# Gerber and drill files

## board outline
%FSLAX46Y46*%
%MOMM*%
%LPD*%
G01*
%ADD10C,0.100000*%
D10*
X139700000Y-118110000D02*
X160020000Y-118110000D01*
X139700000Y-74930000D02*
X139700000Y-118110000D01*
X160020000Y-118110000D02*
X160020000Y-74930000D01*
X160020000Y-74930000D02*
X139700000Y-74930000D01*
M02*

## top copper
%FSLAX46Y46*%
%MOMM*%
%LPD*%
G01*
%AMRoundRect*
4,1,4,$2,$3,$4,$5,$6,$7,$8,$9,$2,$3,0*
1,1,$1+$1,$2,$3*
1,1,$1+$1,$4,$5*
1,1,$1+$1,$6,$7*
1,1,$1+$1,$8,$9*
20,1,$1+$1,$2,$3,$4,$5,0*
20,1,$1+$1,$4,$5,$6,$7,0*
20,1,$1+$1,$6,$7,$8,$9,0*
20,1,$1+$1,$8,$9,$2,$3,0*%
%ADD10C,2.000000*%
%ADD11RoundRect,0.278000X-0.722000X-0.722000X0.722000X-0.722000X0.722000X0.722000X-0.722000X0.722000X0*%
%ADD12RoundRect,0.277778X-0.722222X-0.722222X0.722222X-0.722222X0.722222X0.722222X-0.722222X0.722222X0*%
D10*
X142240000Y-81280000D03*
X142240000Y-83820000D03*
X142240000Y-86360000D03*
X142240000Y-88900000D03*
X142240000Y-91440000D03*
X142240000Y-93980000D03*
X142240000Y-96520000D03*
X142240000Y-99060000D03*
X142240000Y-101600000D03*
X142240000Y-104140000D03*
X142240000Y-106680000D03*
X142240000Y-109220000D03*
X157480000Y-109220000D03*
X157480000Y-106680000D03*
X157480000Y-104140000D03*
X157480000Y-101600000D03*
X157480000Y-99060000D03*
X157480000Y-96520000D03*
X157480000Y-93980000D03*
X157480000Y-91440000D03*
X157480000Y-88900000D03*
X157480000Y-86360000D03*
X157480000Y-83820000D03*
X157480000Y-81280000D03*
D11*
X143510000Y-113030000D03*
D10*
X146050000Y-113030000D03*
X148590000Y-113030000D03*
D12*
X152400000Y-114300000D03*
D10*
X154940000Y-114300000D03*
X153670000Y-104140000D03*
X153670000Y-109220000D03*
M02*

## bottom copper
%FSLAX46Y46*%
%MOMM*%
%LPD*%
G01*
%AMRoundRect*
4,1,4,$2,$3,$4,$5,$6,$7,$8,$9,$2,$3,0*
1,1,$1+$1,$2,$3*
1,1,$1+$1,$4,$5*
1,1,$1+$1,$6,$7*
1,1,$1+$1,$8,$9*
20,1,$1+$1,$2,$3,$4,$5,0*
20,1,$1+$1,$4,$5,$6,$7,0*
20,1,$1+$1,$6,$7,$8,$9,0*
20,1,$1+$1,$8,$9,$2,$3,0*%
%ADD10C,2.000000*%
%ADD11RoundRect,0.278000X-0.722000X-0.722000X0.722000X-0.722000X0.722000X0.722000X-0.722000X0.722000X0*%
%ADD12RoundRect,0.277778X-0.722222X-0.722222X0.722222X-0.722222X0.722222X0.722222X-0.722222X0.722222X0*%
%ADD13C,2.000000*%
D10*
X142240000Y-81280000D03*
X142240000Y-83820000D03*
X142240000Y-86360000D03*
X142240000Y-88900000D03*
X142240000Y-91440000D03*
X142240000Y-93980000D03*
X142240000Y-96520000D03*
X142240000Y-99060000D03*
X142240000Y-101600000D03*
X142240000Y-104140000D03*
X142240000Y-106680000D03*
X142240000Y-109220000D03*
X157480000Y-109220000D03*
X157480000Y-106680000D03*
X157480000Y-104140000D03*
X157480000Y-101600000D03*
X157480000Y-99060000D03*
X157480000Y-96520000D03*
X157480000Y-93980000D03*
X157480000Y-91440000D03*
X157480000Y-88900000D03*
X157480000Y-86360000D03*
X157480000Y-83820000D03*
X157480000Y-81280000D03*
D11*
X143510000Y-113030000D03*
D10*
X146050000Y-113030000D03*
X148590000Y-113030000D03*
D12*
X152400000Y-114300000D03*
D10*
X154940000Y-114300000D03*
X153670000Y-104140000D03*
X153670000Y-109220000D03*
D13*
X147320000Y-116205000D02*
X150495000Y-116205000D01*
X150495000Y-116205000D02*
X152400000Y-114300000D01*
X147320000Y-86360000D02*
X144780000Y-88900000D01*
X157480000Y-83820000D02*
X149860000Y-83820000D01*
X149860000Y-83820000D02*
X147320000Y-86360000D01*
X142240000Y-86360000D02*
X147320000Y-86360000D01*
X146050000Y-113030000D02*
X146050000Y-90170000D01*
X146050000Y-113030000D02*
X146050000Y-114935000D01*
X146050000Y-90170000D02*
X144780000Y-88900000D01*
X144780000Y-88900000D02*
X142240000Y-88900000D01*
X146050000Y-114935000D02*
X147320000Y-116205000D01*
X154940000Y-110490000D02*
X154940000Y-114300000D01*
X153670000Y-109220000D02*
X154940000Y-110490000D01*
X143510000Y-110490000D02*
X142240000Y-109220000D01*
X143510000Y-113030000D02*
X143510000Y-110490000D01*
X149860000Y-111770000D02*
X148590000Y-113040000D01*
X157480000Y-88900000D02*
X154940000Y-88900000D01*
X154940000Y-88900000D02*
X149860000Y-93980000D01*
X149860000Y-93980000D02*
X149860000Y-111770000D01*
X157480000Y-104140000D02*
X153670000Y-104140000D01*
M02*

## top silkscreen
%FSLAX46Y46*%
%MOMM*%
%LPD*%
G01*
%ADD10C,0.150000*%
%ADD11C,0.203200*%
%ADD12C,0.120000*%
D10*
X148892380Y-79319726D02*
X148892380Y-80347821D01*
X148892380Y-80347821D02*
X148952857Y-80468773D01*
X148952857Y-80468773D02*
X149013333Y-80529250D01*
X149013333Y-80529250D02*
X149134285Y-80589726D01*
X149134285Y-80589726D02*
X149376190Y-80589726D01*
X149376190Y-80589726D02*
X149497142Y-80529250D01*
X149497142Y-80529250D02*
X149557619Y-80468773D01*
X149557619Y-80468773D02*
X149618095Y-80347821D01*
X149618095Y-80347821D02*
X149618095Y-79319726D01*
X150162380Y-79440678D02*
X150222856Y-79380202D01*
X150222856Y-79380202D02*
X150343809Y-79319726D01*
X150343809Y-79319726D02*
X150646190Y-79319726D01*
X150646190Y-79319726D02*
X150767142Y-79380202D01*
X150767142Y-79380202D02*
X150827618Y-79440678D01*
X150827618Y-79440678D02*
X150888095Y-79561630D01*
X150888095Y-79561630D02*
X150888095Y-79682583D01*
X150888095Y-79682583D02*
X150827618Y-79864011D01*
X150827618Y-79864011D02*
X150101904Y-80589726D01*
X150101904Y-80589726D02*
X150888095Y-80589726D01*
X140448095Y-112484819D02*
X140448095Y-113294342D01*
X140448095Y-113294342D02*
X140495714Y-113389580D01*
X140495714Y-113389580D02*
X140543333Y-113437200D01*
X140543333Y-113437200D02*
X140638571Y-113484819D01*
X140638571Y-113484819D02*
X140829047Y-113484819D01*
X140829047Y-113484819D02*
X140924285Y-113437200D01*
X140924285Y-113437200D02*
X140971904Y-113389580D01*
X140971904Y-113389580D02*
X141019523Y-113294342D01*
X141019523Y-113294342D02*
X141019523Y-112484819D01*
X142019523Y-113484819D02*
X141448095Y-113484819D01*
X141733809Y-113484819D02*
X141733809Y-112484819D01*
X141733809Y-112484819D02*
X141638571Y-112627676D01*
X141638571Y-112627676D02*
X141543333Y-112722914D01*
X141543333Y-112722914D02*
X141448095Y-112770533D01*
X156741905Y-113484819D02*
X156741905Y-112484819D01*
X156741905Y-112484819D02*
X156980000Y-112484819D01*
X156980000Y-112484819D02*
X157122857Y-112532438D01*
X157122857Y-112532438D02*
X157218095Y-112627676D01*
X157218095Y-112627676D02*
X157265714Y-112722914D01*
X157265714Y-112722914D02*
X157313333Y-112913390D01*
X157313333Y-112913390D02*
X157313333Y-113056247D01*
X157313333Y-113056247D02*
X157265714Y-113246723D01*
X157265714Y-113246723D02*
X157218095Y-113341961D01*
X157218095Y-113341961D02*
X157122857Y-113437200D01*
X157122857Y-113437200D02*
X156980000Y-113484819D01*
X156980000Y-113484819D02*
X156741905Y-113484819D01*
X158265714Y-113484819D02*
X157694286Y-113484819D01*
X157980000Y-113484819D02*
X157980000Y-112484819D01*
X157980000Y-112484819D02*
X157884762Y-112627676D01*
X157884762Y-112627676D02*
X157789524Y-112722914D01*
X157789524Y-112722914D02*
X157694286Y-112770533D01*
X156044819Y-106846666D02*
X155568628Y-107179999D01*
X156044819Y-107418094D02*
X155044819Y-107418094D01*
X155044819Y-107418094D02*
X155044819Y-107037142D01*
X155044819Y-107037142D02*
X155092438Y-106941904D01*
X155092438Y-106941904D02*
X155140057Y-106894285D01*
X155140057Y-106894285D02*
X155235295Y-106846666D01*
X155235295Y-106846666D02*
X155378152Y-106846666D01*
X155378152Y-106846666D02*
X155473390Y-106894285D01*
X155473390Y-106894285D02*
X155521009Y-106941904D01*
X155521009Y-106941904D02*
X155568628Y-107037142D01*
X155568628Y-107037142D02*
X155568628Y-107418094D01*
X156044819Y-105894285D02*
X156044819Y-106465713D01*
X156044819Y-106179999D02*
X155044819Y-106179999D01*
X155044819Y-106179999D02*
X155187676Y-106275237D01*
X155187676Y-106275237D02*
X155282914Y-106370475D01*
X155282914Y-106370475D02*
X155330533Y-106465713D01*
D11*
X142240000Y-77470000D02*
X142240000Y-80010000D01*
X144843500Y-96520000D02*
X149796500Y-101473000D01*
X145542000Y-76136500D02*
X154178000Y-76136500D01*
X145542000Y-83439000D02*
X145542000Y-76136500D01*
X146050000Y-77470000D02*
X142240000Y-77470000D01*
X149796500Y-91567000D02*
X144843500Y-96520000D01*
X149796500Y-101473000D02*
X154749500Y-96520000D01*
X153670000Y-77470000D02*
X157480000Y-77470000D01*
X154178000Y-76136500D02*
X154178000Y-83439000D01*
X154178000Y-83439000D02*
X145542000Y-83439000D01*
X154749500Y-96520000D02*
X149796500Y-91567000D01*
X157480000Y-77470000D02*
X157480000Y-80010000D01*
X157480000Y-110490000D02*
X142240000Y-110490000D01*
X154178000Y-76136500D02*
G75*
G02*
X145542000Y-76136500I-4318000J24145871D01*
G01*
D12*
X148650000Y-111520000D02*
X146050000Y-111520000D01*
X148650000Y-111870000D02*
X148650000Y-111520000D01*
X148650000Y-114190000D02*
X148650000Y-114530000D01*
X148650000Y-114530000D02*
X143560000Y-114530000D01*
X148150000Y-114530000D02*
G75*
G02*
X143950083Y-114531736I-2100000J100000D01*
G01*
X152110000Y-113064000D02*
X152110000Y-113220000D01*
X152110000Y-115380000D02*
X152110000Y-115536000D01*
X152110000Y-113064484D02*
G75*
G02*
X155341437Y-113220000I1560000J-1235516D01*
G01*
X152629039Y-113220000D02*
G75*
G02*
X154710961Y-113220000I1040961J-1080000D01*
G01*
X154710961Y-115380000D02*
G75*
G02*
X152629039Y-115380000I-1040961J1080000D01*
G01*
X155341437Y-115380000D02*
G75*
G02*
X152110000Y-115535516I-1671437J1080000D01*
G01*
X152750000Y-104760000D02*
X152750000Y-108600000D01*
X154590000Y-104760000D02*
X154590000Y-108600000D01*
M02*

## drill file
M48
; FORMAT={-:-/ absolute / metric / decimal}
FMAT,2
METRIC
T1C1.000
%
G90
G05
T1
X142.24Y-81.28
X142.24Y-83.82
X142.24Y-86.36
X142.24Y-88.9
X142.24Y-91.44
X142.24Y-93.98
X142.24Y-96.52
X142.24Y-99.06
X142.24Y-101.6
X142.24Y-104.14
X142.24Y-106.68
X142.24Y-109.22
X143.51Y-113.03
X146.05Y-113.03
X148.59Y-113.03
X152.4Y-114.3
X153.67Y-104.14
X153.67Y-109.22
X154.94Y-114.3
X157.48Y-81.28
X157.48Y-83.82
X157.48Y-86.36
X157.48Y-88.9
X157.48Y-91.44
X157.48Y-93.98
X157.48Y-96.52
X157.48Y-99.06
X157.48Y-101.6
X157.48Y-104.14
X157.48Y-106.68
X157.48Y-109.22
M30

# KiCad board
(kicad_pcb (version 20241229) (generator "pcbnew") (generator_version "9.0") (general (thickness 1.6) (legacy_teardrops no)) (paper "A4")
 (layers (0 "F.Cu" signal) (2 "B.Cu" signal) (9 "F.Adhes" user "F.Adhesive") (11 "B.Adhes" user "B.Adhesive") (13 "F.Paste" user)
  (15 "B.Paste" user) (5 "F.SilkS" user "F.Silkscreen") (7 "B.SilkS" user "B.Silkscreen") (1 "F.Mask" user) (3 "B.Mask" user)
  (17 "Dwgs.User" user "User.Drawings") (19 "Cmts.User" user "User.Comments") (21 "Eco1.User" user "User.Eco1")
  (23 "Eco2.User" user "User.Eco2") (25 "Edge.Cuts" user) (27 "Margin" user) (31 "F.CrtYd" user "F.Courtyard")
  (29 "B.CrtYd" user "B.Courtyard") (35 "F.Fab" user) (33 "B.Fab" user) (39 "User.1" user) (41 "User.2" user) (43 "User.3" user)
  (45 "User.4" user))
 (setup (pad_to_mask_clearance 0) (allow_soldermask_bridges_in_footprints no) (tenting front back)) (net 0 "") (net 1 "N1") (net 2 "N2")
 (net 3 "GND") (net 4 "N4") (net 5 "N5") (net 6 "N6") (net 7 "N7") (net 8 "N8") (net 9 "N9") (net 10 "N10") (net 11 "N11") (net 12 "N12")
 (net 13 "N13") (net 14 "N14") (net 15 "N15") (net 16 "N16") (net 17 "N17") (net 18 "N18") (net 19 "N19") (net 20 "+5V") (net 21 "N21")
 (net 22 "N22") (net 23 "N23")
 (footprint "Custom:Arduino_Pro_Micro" (layer "F.Cu") (at 149.86 93.98)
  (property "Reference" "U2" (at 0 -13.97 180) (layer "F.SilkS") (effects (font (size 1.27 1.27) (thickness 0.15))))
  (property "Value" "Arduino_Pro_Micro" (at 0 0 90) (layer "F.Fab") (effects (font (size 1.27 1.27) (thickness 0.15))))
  (fp_line (start -7.62 -16.51) (end -7.62 -13.97) (stroke (width 0.2032) (type solid)) (layer "F.SilkS"))
  (fp_line (start -5.0165 2.54) (end -0.0635 7.493) (stroke (width 0.2032) (type solid)) (layer "F.SilkS"))
  (fp_line (start -4.318 -17.8435) (end 4.318 -17.8435) (stroke (width 0.2032) (type solid)) (layer "F.SilkS"))
  (fp_line (start -4.318 -10.541) (end -4.318 -17.8435) (stroke (width 0.2032) (type solid)) (layer "F.SilkS"))
  (fp_line (start -3.81 -16.51) (end -7.62 -16.51) (stroke (width 0.2032) (type solid)) (layer "F.SilkS"))
  (fp_line (start -0.0635 -2.413) (end -5.0165 2.54) (stroke (width 0.2032) (type solid)) (layer "F.SilkS"))
  (fp_line (start -0.0635 7.493) (end 4.8895 2.54) (stroke (width 0.2032) (type solid)) (layer "F.SilkS"))
  (fp_line (start 3.81 -16.51) (end 7.62 -16.51) (stroke (width 0.2032) (type solid)) (layer "F.SilkS"))
  (fp_line (start 4.318 -17.8435) (end 4.318 -10.541) (stroke (width 0.2032) (type solid)) (layer "F.SilkS"))
  (fp_line (start 4.318 -10.541) (end -4.318 -10.541) (stroke (width 0.2032) (type solid)) (layer "F.SilkS"))
  (fp_line (start 4.8895 2.54) (end -0.0635 -2.413) (stroke (width 0.2032) (type solid)) (layer "F.SilkS"))
  (fp_line (start 7.62 -16.51) (end 7.62 -13.97) (stroke (width 0.2032) (type solid)) (layer "F.SilkS"))
  (fp_line (start 7.62 16.51) (end -7.62 16.51) (stroke (width 0.2032) (type solid)) (layer "F.SilkS"))
  (fp_arc (start 4.318 -17.8435) (mid 0 -17.460445) (end -4.318 -17.8435) (stroke (width 0.2032) (type solid)) (layer "F.SilkS"))
  (pad "1" thru_hole circle (at -7.62 -12.7) (size 2 2) (drill 1) (layers "*.Cu" "*.Mask") (remove_unused_layers no) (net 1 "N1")
   (thermal_bridge_angle 0))
  (pad "2" thru_hole circle (at -7.62 -10.16) (size 2 2) (drill 1) (layers "*.Cu" "*.Mask") (remove_unused_layers no) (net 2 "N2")
   (thermal_bridge_angle 0))
  (pad "3" thru_hole circle (at -7.62 -7.62) (size 2 2) (drill 1) (layers "*.Cu" "*.Mask") (remove_unused_layers no) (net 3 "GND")
   (thermal_bridge_angle 0))
  (pad "4" thru_hole circle (at -7.62 -5.08) (size 2 2) (drill 1) (layers "*.Cu" "*.Mask") (remove_unused_layers no) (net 3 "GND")
   (thermal_bridge_angle 0))
  (pad "5" thru_hole circle (at -7.62 -2.54) (size 2 2) (drill 1) (layers "*.Cu" "*.Mask") (remove_unused_layers no) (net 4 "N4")
   (thermal_bridge_angle 0))
  (pad "6" thru_hole circle (at -7.62 0) (size 2 2) (drill 1) (layers "*.Cu" "*.Mask") (remove_unused_layers no) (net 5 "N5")
   (thermal_bridge_angle 0))
  (pad "7" thru_hole circle (at -7.62 2.54) (size 2 2) (drill 1) (layers "*.Cu" "*.Mask") (remove_unused_layers no) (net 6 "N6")
   (thermal_bridge_angle 0))
  (pad "8" thru_hole circle (at -7.62 5.08) (size 2 2) (drill 1) (layers "*.Cu" "*.Mask") (remove_unused_layers no) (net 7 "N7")
   (thermal_bridge_angle 0))
  (pad "9" thru_hole circle (at -7.62 7.62) (size 2 2) (drill 1) (layers "*.Cu" "*.Mask") (remove_unused_layers no) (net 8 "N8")
   (thermal_bridge_angle 0))
  (pad "10" thru_hole circle (at -7.62 10.16) (size 2 2) (drill 1) (layers "*.Cu" "*.Mask") (remove_unused_layers no) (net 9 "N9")
   (thermal_bridge_angle 0))
  (pad "11" thru_hole circle (at -7.62 12.7) (size 2 2) (drill 1) (layers "*.Cu" "*.Mask") (remove_unused_layers no) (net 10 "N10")
   (thermal_bridge_angle 0))
  (pad "12" thru_hole circle (at -7.62 15.24) (size 2 2) (drill 1) (layers "*.Cu" "*.Mask") (remove_unused_layers no) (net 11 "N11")
   (thermal_bridge_angle 0))
  (pad "13" thru_hole circle (at 7.62 15.24) (size 2 2) (drill 1) (layers "*.Cu" "*.Mask") (remove_unused_layers no) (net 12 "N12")
   (thermal_bridge_angle 0))
  (pad "14" thru_hole circle (at 7.62 12.7) (size 2 2) (drill 1) (layers "*.Cu" "*.Mask") (remove_unused_layers no) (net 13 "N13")
   (thermal_bridge_angle 0))
  (pad "15" thru_hole circle (at 7.62 10.16) (size 2 2) (drill 1) (layers "*.Cu" "*.Mask") (remove_unused_layers no) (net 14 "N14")
   (thermal_bridge_angle 0))
  (pad "16" thru_hole circle (at 7.62 7.62) (size 2 2) (drill 1) (layers "*.Cu" "*.Mask") (remove_unused_layers no) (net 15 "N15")
   (thermal_bridge_angle 0))
  (pad "17" thru_hole circle (at 7.62 5.08) (size 2 2) (drill 1) (layers "*.Cu" "*.Mask") (remove_unused_layers no) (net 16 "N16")
   (thermal_bridge_angle 0))
  (pad "18" thru_hole circle (at 7.62 2.54) (size 2 2) (drill 1) (layers "*.Cu" "*.Mask") (remove_unused_layers no) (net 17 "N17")
   (thermal_bridge_angle 0))
  (pad "19" thru_hole circle (at 7.62 0) (size 2 2) (drill 1) (layers "*.Cu" "*.Mask") (remove_unused_layers no) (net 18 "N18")
   (thermal_bridge_angle 0))
  (pad "20" thru_hole circle (at 7.62 -2.54) (size 2 2) (drill 1) (layers "*.Cu" "*.Mask") (remove_unused_layers no) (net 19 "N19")
   (thermal_bridge_angle 0))
  (pad "21" thru_hole circle (at 7.62 -5.08) (size 2 2) (drill 1) (layers "*.Cu" "*.Mask") (remove_unused_layers no) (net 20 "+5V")
   (thermal_bridge_angle 0))
  (pad "22" thru_hole circle (at 7.62 -7.62) (size 2 2) (drill 1) (layers "*.Cu" "*.Mask") (remove_unused_layers no) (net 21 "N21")
   (thermal_bridge_angle 0))
  (pad "23" thru_hole circle (at 7.62 -10.16) (size 2 2) (drill 1) (layers "*.Cu" "*.Mask") (remove_unused_layers no) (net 3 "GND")
   (thermal_bridge_angle 0))
  (pad "24" thru_hole circle (at 7.62 -12.7) (size 2 2) (drill 1) (layers "*.Cu" "*.Mask") (remove_unused_layers no) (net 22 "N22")
   (thermal_bridge_angle 0)))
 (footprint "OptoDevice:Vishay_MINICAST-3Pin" (layer "F.Cu") (at 143.51 113.03)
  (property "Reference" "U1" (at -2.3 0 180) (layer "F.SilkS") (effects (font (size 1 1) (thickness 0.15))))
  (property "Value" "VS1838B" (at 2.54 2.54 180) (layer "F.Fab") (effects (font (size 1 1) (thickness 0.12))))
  (fp_line (start 5.14 -1.51) (end 2.54 -1.51) (stroke (width 0.12) (type solid)) (layer "F.SilkS"))
  (fp_line (start 5.14 -1.16) (end 5.14 -1.51) (stroke (width 0.12) (type solid)) (layer "F.SilkS"))
  (fp_line (start 5.14 1.16) (end 5.14 1.5) (stroke (width 0.12) (type solid)) (layer "F.SilkS"))
  (fp_line (start 5.14 1.5) (end 0.05 1.5) (stroke (width 0.12) (type solid)) (layer "F.SilkS"))
  (fp_arc (start 4.64 1.5) (mid 2.540869 3.502379) (end 0.440083 1.501736) (stroke (width 0.12) (type solid)) (layer "F.SilkS"))
  (pad "1" thru_hole roundrect (at 0 0) (size 2 2) (drill 1) (layers "*.Cu" "*.Mask") (remove_unused_layers no) (roundrect_rratio 0.139)
   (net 11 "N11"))
  (pad "2" thru_hole circle (at 2.54 0) (size 2 2) (drill 1) (layers "*.Cu" "*.Mask") (remove_unused_layers no) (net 3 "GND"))
  (pad "3" thru_hole circle (at 5.08 0) (size 2 2) (drill 1) (layers "*.Cu" "*.Mask") (remove_unused_layers no) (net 20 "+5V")))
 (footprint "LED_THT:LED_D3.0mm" (layer "F.Cu") (at 152.4 114.3)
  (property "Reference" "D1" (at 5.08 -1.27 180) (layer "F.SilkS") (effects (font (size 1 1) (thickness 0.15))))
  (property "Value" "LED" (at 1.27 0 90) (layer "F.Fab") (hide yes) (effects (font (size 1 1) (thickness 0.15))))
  (fp_line (start -0.29 -1.236) (end -0.29 -1.08) (stroke (width 0.12) (type solid)) (layer "F.SilkS"))
  (fp_line (start -0.29 1.08) (end -0.29 1.236) (stroke (width 0.12) (type solid)) (layer "F.SilkS"))
  (fp_arc (start -0.29 -1.235516) (mid 1.36566 -1.987699) (end 2.941437 -1.08) (stroke (width 0.12) (type solid)) (layer "F.SilkS"))
  (fp_arc (start 0.229039 -1.08) (mid 1.27 -1.5) (end 2.310961 -1.08) (stroke (width 0.12) (type solid)) (layer "F.SilkS"))
  (fp_arc (start 2.310961 1.08) (mid 1.27 1.5) (end 0.229039 1.08) (stroke (width 0.12) (type solid)) (layer "F.SilkS"))
  (fp_arc (start 2.941437 1.08) (mid 1.36566 1.987699) (end -0.29 1.235516) (stroke (width 0.12) (type solid)) (layer "F.SilkS"))
  (pad "1" thru_hole roundrect (at 0 0) (size 2 2) (drill 1) (layers "*.Cu" "*.Mask") (remove_unused_layers no)
   (roundrect_rratio 0.1388888889) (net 3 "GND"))
  (pad "2" thru_hole circle (at 2.54 0) (size 2 2) (drill 1) (layers "*.Cu" "*.Mask") (remove_unused_layers no) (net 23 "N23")))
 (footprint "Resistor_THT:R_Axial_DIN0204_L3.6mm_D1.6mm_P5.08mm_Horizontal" (layer "F.Cu") (at 153.67 104.14 -90)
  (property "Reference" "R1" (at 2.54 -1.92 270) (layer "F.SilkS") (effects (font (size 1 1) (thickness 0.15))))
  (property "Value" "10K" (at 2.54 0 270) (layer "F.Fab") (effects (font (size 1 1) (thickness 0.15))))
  (fp_line (start 0.62 0.92) (end 4.46 0.92) (stroke (width 0.12) (type solid)) (layer "F.SilkS"))
  (fp_line (start 0.62 -0.92) (end 4.46 -0.92) (stroke (width 0.12) (type solid)) (layer "F.SilkS"))
  (pad "1" thru_hole circle (at 0 0 270) (size 2 2) (drill 1) (layers "*.Cu" "*.Mask") (remove_unused_layers no) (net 14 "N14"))
  (pad "2" thru_hole circle (at 5.08 0 270) (size 2 2) (drill 1) (layers "*.Cu" "*.Mask") (remove_unused_layers no) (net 23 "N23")))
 (gr_line (start 139.7 118.11) (end 160.02 118.11) (stroke (width 0.1) (type solid)) (layer "Edge.Cuts"))
 (gr_line (start 139.7 74.93) (end 139.7 118.11) (stroke (width 0.1) (type default)) (layer "Edge.Cuts"))
 (gr_line (start 160.02 118.11) (end 160.02 74.93) (stroke (width 0.1) (type default)) (layer "Edge.Cuts"))
 (gr_line (start 160.02 74.93) (end 139.7 74.93) (stroke (width 0.1) (type solid)) (layer "Edge.Cuts"))
 (segment (start 147.32 116.205) (end 150.495 116.205) (width 2) (layer "B.Cu") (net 3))
 (segment (start 150.495 116.205) (end 152.4 114.3) (width 2) (layer "B.Cu") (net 3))
 (segment (start 147.32 86.36) (end 144.78 88.9) (width 2) (layer "B.Cu") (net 3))
 (segment (start 157.48 83.82) (end 149.86 83.82) (width 2) (layer "B.Cu") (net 3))
 (segment (start 149.86 83.82) (end 147.32 86.36) (width 2) (layer "B.Cu") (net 3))
 (segment (start 142.24 86.36) (end 147.32 86.36) (width 2) (layer "B.Cu") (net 3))
 (segment (start 146.05 113.03) (end 146.05 90.17) (width 2) (layer "B.Cu") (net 3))
 (segment (start 146.05 113.03) (end 146.05 114.935) (width 2) (layer "B.Cu") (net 3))
 (segment (start 146.05 90.17) (end 144.78 88.9) (width 2) (layer "B.Cu") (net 3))
 (segment (start 144.78 88.9) (end 142.24 88.9) (width 2) (layer "B.Cu") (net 3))
 (segment (start 146.05 114.935) (end 147.32 116.205) (width 2) (layer "B.Cu") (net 3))
 (segment (start 154.94 110.49) (end 154.94 114.3) (width 2) (layer "B.Cu") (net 23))
 (segment (start 153.67 109.22) (end 154.94 110.49) (width 2) (layer "B.Cu") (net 23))
 (segment (start 143.51 110.49) (end 142.24 109.22) (width 2) (layer "B.Cu") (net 11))
 (segment (start 143.51 113.03) (end 143.51 110.49) (width 2) (layer "B.Cu") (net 11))
 (segment (start 149.86 111.77) (end 148.59 113.04) (width 2) (layer "B.Cu") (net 20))
 (segment (start 157.48 88.9) (end 154.94 88.9) (width 2) (layer "B.Cu") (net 20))
 (segment (start 154.94 88.9) (end 149.86 93.98) (width 2) (layer "B.Cu") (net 20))
 (segment (start 149.86 93.98) (end 149.86 111.77) (width 2) (layer "B.Cu") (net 20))
 (segment (start 157.48 104.14) (end 153.67 104.14) (width 2) (layer "B.Cu") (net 14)))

